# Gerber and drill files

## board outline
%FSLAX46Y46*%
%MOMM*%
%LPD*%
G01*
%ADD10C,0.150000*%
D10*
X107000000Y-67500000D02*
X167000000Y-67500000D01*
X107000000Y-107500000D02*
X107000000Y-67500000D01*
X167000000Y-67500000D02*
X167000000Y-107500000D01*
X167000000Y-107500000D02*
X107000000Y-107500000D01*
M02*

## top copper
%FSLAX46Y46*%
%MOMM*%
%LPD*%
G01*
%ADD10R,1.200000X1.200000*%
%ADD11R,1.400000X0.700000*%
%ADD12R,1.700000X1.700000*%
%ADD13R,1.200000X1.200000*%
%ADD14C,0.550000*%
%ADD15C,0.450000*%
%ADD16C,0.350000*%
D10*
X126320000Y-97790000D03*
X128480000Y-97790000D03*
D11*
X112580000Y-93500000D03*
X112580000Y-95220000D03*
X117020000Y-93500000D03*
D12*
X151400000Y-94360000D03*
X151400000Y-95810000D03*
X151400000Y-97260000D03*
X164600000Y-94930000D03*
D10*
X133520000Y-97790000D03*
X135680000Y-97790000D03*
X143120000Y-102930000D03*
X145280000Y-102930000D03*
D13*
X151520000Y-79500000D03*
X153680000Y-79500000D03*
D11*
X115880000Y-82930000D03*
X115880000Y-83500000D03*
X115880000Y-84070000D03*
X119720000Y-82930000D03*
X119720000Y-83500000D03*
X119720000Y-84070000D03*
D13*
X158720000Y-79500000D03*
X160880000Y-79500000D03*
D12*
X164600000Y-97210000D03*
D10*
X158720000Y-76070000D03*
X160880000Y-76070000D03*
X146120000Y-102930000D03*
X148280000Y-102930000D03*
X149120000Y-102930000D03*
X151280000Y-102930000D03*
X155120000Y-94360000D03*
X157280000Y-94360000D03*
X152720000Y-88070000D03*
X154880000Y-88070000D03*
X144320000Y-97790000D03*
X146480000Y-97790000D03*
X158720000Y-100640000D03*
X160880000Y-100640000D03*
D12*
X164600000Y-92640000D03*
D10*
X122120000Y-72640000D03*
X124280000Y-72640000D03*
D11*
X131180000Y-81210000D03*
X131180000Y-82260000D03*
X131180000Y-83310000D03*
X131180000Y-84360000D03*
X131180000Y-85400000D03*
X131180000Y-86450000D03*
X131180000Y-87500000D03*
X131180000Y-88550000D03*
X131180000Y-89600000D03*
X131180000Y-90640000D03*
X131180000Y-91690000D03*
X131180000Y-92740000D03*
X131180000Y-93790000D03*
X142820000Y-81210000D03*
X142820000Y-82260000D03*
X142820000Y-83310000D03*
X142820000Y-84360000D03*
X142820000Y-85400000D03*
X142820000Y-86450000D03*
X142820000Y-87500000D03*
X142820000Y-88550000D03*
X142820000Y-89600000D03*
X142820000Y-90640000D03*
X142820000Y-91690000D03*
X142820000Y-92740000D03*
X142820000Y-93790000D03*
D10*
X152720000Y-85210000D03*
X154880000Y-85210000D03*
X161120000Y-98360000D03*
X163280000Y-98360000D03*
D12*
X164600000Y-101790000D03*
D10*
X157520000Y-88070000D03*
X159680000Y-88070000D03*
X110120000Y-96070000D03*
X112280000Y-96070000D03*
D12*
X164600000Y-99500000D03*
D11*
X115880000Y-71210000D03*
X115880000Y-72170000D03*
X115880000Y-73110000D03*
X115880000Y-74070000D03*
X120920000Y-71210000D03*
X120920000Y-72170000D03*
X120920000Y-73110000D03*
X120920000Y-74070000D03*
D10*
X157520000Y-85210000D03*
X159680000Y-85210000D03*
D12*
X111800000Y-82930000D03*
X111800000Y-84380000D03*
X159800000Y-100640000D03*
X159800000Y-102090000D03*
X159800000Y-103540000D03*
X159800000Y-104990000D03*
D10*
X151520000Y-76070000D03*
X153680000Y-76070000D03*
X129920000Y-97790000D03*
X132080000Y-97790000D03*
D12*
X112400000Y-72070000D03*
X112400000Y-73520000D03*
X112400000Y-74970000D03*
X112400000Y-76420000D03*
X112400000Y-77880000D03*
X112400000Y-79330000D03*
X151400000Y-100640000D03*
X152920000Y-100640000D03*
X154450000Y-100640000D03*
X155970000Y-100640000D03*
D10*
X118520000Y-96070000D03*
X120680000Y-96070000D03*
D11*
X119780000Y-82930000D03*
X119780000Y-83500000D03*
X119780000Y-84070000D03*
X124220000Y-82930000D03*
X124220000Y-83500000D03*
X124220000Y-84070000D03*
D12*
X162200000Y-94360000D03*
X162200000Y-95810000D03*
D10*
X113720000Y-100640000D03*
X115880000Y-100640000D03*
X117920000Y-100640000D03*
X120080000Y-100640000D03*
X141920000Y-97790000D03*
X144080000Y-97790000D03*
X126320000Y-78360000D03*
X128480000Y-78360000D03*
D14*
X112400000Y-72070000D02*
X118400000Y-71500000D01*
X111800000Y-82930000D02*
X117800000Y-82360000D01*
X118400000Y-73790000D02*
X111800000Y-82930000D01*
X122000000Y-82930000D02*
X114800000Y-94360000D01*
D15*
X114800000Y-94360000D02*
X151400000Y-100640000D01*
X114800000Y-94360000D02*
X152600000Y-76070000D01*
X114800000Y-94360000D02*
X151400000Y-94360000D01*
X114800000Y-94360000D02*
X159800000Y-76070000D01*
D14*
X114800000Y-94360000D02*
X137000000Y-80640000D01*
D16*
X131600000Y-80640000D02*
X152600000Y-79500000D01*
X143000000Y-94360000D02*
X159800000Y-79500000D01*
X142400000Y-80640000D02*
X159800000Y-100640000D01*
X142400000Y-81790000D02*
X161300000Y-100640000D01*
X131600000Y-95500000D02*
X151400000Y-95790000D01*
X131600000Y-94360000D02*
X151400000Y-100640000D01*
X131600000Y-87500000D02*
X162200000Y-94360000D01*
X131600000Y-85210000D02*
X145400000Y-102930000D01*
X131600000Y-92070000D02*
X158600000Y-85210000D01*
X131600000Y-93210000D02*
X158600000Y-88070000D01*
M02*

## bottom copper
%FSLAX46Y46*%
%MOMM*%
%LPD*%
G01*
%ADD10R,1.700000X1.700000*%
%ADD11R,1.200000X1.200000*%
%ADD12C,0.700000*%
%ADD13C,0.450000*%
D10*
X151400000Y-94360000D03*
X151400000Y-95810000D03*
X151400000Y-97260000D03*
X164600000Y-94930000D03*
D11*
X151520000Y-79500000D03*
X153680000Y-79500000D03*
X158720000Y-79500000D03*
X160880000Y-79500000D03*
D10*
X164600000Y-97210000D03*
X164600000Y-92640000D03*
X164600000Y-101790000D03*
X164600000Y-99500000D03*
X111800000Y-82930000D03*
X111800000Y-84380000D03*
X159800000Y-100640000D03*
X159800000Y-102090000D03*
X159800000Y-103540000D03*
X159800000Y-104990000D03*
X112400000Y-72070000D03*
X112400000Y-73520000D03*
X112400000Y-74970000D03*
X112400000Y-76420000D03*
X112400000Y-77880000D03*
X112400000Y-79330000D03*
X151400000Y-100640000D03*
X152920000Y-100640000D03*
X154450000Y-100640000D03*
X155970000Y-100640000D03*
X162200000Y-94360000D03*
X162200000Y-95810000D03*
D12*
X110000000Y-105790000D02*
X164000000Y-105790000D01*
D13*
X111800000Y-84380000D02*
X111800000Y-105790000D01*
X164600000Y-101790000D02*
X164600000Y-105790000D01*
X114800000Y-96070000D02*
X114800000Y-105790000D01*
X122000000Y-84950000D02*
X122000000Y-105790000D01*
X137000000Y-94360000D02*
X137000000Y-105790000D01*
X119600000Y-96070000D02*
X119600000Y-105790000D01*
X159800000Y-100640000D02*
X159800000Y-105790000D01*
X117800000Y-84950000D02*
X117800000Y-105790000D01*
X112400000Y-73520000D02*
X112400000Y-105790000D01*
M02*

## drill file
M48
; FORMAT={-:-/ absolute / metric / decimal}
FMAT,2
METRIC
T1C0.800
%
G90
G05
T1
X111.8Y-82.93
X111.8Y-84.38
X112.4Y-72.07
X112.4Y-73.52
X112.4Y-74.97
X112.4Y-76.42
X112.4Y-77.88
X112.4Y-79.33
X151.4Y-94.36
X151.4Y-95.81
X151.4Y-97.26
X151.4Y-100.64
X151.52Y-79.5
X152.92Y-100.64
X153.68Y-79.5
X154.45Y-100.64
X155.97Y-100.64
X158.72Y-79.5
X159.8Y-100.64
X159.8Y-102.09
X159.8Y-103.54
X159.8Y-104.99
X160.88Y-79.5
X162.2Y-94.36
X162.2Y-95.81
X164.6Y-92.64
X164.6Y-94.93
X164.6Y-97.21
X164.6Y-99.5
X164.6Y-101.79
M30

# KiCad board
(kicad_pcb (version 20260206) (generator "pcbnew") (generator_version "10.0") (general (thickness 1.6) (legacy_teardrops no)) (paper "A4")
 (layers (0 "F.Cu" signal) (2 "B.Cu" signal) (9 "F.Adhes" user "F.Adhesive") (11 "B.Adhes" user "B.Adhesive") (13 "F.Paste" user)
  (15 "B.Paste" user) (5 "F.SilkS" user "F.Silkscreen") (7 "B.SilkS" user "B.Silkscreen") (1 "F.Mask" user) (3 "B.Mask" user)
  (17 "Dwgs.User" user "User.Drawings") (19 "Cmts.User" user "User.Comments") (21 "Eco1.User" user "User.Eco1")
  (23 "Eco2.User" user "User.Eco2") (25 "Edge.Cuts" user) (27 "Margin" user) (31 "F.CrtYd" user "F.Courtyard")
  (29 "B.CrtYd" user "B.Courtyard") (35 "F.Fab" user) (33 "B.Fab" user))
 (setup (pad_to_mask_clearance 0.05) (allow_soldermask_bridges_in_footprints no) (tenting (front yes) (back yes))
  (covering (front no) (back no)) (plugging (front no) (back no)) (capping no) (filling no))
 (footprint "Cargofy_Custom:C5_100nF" (layer "F.Cu") (at 127.4 97.79)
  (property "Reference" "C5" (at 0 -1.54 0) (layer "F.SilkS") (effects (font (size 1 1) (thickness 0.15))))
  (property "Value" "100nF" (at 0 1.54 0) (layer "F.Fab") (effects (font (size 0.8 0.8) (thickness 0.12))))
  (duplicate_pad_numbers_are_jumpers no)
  (pad "1" smd rect (at -1.08 0) (size 1.2 1.2) (layers "F.Cu" "F.Mask" "F.Paste") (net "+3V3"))
  (pad "2" smd rect (at 1.08 0) (size 1.2 1.2) (layers "F.Cu" "F.Mask" "F.Paste") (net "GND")))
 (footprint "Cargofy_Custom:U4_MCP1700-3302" (layer "F.Cu") (at 114.8 94.36)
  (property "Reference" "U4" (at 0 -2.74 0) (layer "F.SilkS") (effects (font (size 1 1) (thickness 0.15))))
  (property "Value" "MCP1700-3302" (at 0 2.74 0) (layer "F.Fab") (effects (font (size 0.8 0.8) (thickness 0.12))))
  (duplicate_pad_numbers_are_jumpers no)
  (pad "1" smd rect (at -2.22 -0.86) (size 1.4 0.7) (layers "F.Cu" "F.Mask" "F.Paste") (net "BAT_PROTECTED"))
  (pad "2" smd rect (at -2.22 0.86) (size 1.4 0.7) (layers "F.Cu" "F.Mask" "F.Paste") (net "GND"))
  (pad "3" smd rect (at 2.22 -0.86) (size 1.4 0.7) (layers "F.Cu" "F.Mask" "F.Paste") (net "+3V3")))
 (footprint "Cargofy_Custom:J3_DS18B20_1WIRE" (layer "F.Cu") (at 151.4 94.36)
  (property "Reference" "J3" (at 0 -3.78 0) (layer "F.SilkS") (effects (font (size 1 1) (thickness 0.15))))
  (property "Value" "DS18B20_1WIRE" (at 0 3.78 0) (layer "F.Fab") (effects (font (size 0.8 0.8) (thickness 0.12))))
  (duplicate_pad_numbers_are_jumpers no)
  (pad "1" thru_hole rect (at 0 0) (size 1.7 1.7) (drill 0.8) (layers "*.Cu" "*.Mask") (remove_unused_layers no) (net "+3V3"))
  (pad "2" thru_hole rect (at 0 1.45) (size 1.7 1.7) (drill 0.8) (layers "*.Cu" "*.Mask") (remove_unused_layers no) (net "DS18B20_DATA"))
  (pad "3" thru_hole rect (at 0 2.9) (size 1.7 1.7) (drill 0.8) (layers "*.Cu" "*.Mask") (remove_unused_layers no) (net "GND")))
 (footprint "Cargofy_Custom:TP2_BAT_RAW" (layer "F.Cu") (at 164.6 94.93)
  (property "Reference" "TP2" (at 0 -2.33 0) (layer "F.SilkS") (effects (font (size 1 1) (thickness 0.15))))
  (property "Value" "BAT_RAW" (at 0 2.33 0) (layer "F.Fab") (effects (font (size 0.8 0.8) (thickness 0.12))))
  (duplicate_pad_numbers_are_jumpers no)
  (pad "1" thru_hole rect (at 0 0) (size 1.7 1.7) (drill 0.8) (layers "*.Cu" "*.Mask") (remove_unused_layers no) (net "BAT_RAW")))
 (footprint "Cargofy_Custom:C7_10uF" (layer "F.Cu") (at 134.6 97.79)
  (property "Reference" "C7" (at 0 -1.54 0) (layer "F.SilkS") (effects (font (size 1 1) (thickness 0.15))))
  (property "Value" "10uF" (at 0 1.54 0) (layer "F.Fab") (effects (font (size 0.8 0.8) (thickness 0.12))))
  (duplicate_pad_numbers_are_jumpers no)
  (pad "1" smd rect (at -1.08 0) (size 1.2 1.2) (layers "F.Cu" "F.Mask" "F.Paste") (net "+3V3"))
  (pad "2" smd rect (at 1.08 0) (size 1.2 1.2) (layers "F.Cu" "F.Mask" "F.Paste") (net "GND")))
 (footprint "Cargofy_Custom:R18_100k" (layer "F.Cu") (at 144.2 102.93)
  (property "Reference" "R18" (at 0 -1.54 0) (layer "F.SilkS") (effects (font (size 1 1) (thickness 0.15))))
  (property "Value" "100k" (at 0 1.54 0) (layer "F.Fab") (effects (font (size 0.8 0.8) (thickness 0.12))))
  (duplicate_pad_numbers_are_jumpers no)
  (pad "1" smd rect (at -1.08 0) (size 1.2 1.2) (layers "F.Cu" "F.Mask" "F.Paste") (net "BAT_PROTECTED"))
  (pad "2" smd rect (at 1.08 0) (size 1.2 1.2) (layers "F.Cu" "F.Mask" "F.Paste") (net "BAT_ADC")))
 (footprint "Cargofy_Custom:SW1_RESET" (layer "F.Cu") (at 152.6 79.5)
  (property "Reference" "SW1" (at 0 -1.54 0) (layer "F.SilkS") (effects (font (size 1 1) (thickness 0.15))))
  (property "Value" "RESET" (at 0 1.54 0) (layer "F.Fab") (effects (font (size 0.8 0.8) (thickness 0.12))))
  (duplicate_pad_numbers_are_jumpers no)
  (pad "1" thru_hole rect (at -1.08 0) (size 1.2 1.2) (drill 0.8) (layers "*.Cu" "*.Mask") (remove_unused_layers no) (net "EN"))
  (pad "2" thru_hole rect (at 1.08 0) (size 1.2 1.2) (drill 0.8) (layers "*.Cu" "*.Mask") (remove_unused_layers no) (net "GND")))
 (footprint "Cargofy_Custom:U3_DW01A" (layer "F.Cu") (at 117.8 83.5)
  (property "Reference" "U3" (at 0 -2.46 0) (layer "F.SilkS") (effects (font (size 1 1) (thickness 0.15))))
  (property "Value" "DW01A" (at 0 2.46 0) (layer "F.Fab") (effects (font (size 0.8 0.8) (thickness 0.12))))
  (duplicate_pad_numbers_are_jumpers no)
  (pad "1" smd rect (at -1.92 -0.57) (size 1.4 0.7) (layers "F.Cu" "F.Mask" "F.Paste") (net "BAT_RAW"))
  (pad "2" smd rect (at -1.92 0) (size 1.4 0.7) (layers "F.Cu" "F.Mask" "F.Paste") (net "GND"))
  (pad "3" smd rect (at -1.92 0.57) (size 1.4 0.7) (layers "F.Cu" "F.Mask" "F.Paste") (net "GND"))
  (pad "4" smd rect (at 1.92 -0.57) (size 1.4 0.7) (layers "F.Cu" "F.Mask" "F.Paste") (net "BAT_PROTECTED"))
  (pad "5" smd rect (at 1.92 0) (size 1.4 0.7) (layers "F.Cu" "F.Mask" "F.Paste") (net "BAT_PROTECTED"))
  (pad "6" smd rect (at 1.92 0.57) (size 1.4 0.7) (layers "F.Cu" "F.Mask" "F.Paste") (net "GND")))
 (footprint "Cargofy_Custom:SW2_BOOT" (layer "F.Cu") (at 159.8 79.5)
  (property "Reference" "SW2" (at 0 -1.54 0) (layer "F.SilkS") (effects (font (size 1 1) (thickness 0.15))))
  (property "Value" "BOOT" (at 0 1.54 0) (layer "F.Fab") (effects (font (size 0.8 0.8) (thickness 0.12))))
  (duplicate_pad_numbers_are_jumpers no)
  (pad "1" thru_hole rect (at -1.08 0) (size 1.2 1.2) (drill 0.8) (layers "*.Cu" "*.Mask") (remove_unused_layers no) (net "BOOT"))
  (pad "2" thru_hole rect (at 1.08 0) (size 1.2 1.2) (drill 0.8) (layers "*.Cu" "*.Mask") (remove_unused_layers no) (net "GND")))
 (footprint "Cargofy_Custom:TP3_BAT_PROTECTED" (layer "F.Cu") (at 164.6 97.21)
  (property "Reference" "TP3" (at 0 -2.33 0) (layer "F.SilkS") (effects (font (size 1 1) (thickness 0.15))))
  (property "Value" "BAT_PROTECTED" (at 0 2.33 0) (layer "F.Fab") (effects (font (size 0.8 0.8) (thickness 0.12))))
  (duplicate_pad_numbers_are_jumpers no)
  (pad "1" thru_hole rect (at 0 0) (size 1.7 1.7) (drill 0.8) (layers "*.Cu" "*.Mask") (remove_unused_layers no) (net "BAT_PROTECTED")))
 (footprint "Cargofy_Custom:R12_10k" (layer "F.Cu") (at 159.8 76.07)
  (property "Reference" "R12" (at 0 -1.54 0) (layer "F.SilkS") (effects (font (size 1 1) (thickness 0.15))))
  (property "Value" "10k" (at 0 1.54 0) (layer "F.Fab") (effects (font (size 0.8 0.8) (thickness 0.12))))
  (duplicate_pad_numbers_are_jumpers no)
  (pad "1" smd rect (at -1.08 0) (size 1.2 1.2) (layers "F.Cu" "F.Mask" "F.Paste") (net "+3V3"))
  (pad "2" smd rect (at 1.08 0) (size 1.2 1.2) (layers "F.Cu" "F.Mask" "F.Paste") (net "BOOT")))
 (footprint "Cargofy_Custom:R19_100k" (layer "F.Cu") (at 147.2 102.93)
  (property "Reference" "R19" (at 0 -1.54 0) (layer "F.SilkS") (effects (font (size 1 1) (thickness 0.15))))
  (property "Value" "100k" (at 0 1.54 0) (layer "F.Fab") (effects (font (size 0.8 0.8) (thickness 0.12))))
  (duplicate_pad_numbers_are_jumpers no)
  (pad "1" smd rect (at -1.08 0) (size 1.2 1.2) (layers "F.Cu" "F.Mask" "F.Paste") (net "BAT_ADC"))
  (pad "2" smd rect (at 1.08 0) (size 1.2 1.2) (layers "F.Cu" "F.Mask" "F.Paste") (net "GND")))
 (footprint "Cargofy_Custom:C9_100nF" (layer "F.Cu") (at 150.2 102.93)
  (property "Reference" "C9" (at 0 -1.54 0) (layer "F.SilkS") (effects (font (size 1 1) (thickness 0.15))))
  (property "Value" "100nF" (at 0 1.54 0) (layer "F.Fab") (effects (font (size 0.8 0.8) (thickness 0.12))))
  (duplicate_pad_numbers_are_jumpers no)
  (pad "1" smd rect (at -1.08 0) (size 1.2 1.2) (layers "F.Cu" "F.Mask" "F.Paste") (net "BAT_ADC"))
  (pad "2" smd rect (at 1.08 0) (size 1.2 1.2) (layers "F.Cu" "F.Mask" "F.Paste") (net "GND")))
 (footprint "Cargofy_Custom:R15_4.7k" (layer "F.Cu") (at 156.2 94.36)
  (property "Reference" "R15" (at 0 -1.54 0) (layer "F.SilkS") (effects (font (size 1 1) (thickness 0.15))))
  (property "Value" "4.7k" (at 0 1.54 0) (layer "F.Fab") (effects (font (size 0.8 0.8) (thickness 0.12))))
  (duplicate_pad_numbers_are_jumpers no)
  (pad "1" smd rect (at -1.08 0) (size 1.2 1.2) (layers "F.Cu" "F.Mask" "F.Paste") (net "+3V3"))
  (pad "2" smd rect (at 1.08 0) (size 1.2 1.2) (layers "F.Cu" "F.Mask" "F.Paste") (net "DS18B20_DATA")))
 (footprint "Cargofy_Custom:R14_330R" (layer "F.Cu") (at 153.8 88.07)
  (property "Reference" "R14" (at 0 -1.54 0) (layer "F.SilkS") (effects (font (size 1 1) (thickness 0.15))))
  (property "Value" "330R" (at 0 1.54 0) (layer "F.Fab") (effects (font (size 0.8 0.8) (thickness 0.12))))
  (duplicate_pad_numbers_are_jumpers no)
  (pad "1" smd rect (at -1.08 0) (size 1.2 1.2) (layers "F.Cu" "F.Mask" "F.Paste") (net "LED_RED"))
  (pad "2" smd rect (at 1.08 0) (size 1.2 1.2) (layers "F.Cu" "F.Mask" "F.Paste") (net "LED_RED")))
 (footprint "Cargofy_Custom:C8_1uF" (layer "F.Cu") (at 145.4 97.79)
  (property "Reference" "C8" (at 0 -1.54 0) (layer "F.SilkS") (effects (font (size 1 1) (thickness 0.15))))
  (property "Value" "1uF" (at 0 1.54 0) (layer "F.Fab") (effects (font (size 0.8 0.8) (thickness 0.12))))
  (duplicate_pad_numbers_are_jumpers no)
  (pad "1" smd rect (at -1.08 0) (size 1.2 1.2) (layers "F.Cu" "F.Mask" "F.Paste") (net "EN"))
  (pad "2" smd rect (at 1.08 0) (size 1.2 1.2) (layers "F.Cu" "F.Mask" "F.Paste") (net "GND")))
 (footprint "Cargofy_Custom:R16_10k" (layer "F.Cu") (at 159.8 100.64)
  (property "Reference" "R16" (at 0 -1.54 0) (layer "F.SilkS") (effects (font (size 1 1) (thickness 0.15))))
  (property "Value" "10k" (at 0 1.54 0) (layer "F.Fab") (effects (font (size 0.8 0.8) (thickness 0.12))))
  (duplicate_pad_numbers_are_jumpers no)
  (pad "1" smd rect (at -1.08 0) (size 1.2 1.2) (layers "F.Cu" "F.Mask" "F.Paste") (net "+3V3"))
  (pad "2" smd rect (at 1.08 0) (size 1.2 1.2) (layers "F.Cu" "F.Mask" "F.Paste") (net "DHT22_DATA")))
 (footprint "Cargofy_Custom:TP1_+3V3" (layer "F.Cu") (at 164.6 92.64)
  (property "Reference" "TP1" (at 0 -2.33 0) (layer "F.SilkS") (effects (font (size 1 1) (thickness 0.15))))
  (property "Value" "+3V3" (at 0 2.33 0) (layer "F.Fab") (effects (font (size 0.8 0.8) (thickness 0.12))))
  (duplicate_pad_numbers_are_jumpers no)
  (pad "1" thru_hole rect (at 0 0) (size 1.7 1.7) (drill 0.8) (layers "*.Cu" "*.Mask") (remove_unused_layers no) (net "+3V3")))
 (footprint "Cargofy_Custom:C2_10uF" (layer "F.Cu") (at 123.2 72.64)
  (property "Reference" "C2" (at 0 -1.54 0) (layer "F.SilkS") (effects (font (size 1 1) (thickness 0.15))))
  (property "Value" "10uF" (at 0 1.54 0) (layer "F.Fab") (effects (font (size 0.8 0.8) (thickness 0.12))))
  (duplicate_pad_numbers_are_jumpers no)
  (pad "1" smd rect (at -1.08 0) (size 1.2 1.2) (layers "F.Cu" "F.Mask" "F.Paste") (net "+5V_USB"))
  (pad "2" smd rect (at 1.08 0) (size 1.2 1.2) (layers "F.Cu" "F.Mask" "F.Paste") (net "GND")))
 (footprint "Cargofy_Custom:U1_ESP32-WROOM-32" (layer "F.Cu") (at 137 87.5)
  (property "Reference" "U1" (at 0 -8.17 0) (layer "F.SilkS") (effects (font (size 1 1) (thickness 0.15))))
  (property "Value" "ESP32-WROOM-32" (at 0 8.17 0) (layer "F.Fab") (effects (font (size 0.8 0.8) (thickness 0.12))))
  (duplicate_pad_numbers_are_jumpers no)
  (pad "1" smd rect (at -5.82 -6.29) (size 1.4 0.7) (layers "F.Cu" "F.Mask" "F.Paste") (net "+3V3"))
  (pad "2" smd rect (at -5.82 -5.24) (size 1.4 0.7) (layers "F.Cu" "F.Mask" "F.Paste") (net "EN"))
  (pad "3" smd rect (at -5.82 -4.19) (size 1.4 0.7) (layers "F.Cu" "F.Mask" "F.Paste") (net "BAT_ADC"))
  (pad "4" smd rect (at -5.82 -3.14) (size 1.4 0.7) (layers "F.Cu" "F.Mask" "F.Paste") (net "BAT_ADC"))
  (pad "5" smd rect (at -5.82 -2.1) (size 1.4 0.7) (layers "F.Cu" "F.Mask" "F.Paste") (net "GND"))
  (pad "6" smd rect (at -5.82 -1.05) (size 1.4 0.7) (layers "F.Cu" "F.Mask" "F.Paste") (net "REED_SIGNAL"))
  (pad "7" smd rect (at -5.82 0) (size 1.4 0.7) (layers "F.Cu" "F.Mask" "F.Paste") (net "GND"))
  (pad "8" smd rect (at -5.82 1.05) (size 1.4 0.7) (layers "F.Cu" "F.Mask" "F.Paste") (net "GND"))
  (pad "9" smd rect (at -5.82 2.1) (size 1.4 0.7) (layers "F.Cu" "F.Mask" "F.Paste") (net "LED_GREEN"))
  (pad "10" smd rect (at -5.82 3.14) (size 1.4 0.7) (layers "F.Cu" "F.Mask" "F.Paste") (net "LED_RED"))
  (pad "11" smd rect (at -5.82 4.19) (size 1.4 0.7) (layers "F.Cu" "F.Mask" "F.Paste") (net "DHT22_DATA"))
  (pad "12" smd rect (at -5.82 5.24) (size 1.4 0.7) (layers "F.Cu" "F.Mask" "F.Paste") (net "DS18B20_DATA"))
  (pad "13" smd rect (at -5.82 6.29) (size 1.4 0.7) (layers "F.Cu" "F.Mask" "F.Paste") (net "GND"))
  (pad "14" smd rect (at 5.82 -6.29) (size 1.4 0.7) (layers "F.Cu" "F.Mask" "F.Paste") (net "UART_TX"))
  (pad "15" smd rect (at 5.82 -5.24) (size 1.4 0.7) (layers "F.Cu" "F.Mask" "F.Paste") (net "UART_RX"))
  (pad "16" smd rect (at 5.82 -4.19) (size 1.4 0.7) (layers "F.Cu" "F.Mask" "F.Paste") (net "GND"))
  (pad "17" smd rect (at 5.82 -3.14) (size 1.4 0.7) (layers "F.Cu" "F.Mask" "F.Paste") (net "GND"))
  (pad "18" smd rect (at 5.82 -2.1) (size 1.4 0.7) (layers "F.Cu" "F.Mask" "F.Paste") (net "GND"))
  (pad "19" smd rect (at 5.82 -1.05) (size 1.4 0.7) (layers "F.Cu" "F.Mask" "F.Paste") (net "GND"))
  (pad "20" smd rect (at 5.82 0) (size 1.4 0.7) (layers "F.Cu" "F.Mask" "F.Paste") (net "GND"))
  (pad "21" smd rect (at 5.82 1.05) (size 1.4 0.7) (layers "F.Cu" "F.Mask" "F.Paste") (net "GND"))
  (pad "22" smd rect (at 5.82 2.1) (size 1.4 0.7) (layers "F.Cu" "F.Mask" "F.Paste") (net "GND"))
  (pad "23" smd rect (at 5.82 3.14) (size 1.4 0.7) (layers "F.Cu" "F.Mask" "F.Paste") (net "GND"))
  (pad "24" smd rect (at 5.82 4.19) (size 1.4 0.7) (layers "F.Cu" "F.Mask" "F.Paste") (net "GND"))
  (pad "25" smd rect (at 5.82 5.24) (size 1.4 0.7) (layers "F.Cu" "F.Mask" "F.Paste") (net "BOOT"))
  (pad "26" smd rect (at 5.82 6.29) (size 1.4 0.7) (layers "F.Cu" "F.Mask" "F.Paste") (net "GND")))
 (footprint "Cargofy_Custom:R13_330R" (layer "F.Cu") (at 153.8 85.21)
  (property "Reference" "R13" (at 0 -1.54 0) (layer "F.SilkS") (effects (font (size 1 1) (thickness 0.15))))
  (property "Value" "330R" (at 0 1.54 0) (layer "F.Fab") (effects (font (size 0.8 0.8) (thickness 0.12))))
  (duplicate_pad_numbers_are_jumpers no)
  (pad "1" smd rect (at -1.08 0) (size 1.2 1.2) (layers "F.Cu" "F.Mask" "F.Paste") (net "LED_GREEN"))
  (pad "2" smd rect (at 1.08 0) (size 1.2 1.2) (layers "F.Cu" "F.Mask" "F.Paste") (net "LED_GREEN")))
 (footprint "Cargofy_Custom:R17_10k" (layer "F.Cu") (at 162.2 98.36)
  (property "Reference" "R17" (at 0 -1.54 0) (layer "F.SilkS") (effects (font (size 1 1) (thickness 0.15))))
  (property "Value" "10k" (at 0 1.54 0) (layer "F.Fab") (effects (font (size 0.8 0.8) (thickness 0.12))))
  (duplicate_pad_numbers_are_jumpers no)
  (pad "1" smd rect (at -1.08 0) (size 1.2 1.2) (layers "F.Cu" "F.Mask" "F.Paste") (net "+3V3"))
  (pad "2" smd rect (at 1.08 0) (size 1.2 1.2) (layers "F.Cu" "F.Mask" "F.Paste") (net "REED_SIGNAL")))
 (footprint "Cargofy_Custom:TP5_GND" (layer "F.Cu") (at 164.6 101.79)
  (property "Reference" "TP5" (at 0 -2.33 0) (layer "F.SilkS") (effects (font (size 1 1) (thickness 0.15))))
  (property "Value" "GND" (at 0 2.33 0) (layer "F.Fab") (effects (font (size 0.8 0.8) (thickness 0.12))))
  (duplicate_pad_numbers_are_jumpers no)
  (pad "1" thru_hole rect (at 0 0) (size 1.7 1.7) (drill 0.8) (layers "*.Cu" "*.Mask") (remove_unused_layers no) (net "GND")))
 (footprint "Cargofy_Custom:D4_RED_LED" (layer "F.Cu") (at 158.6 88.07)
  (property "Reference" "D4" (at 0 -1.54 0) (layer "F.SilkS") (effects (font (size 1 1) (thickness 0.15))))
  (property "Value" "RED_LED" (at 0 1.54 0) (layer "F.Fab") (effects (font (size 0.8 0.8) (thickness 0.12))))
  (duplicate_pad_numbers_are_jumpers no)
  (pad "1" smd rect (at -1.08 0) (size 1.2 1.2) (layers "F.Cu" "F.Mask" "F.Paste") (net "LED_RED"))
  (pad "2" smd rect (at 1.08 0) (size 1.2 1.2) (layers "F.Cu" "F.Mask" "F.Paste") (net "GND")))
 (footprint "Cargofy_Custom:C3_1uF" (layer "F.Cu") (at 111.2 96.07)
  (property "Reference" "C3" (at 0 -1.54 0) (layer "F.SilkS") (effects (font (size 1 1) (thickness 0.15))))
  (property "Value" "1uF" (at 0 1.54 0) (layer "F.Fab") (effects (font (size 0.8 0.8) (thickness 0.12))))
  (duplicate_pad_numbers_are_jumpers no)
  (pad "1" smd rect (at -1.08 0) (size 1.2 1.2) (layers "F.Cu" "F.Mask" "F.Paste") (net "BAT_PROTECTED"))
  (pad "2" smd rect (at 1.08 0) (size 1.2 1.2) (layers "F.Cu" "F.Mask" "F.Paste") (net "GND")))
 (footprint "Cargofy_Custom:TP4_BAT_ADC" (layer "F.Cu") (at 164.6 99.5)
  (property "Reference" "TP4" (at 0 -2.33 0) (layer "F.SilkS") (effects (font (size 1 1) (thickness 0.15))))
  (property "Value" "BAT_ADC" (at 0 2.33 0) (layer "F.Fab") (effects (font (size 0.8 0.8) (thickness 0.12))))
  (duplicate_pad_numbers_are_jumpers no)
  (pad "1" thru_hole rect (at 0 0) (size 1.7 1.7) (drill 0.8) (layers "*.Cu" "*.Mask") (remove_unused_layers no) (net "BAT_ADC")))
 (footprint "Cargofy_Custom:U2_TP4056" (layer "F.Cu") (at 118.4 72.64)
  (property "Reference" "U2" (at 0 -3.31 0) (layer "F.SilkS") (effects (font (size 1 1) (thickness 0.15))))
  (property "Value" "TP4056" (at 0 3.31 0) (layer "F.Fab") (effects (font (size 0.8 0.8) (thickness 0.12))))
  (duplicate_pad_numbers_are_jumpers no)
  (pad "1" smd rect (at -2.52 -1.43) (size 1.4 0.7) (layers "F.Cu" "F.Mask" "F.Paste") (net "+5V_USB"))
  (pad "2" smd rect (at -2.52 -0.47) (size 1.4 0.7) (layers "F.Cu" "F.Mask" "F.Paste") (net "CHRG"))
  (pad "3" smd rect (at -2.52 0.47) (size 1.4 0.7) (layers "F.Cu" "F.Mask" "F.Paste") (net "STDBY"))
  (pad "4" smd rect (at -2.52 1.43) (size 1.4 0.7) (layers "F.Cu" "F.Mask" "F.Paste") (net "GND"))
  (pad "5" smd rect (at 2.52 -1.43) (size 1.4 0.7) (layers "F.Cu" "F.Mask" "F.Paste") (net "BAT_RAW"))
  (pad "6" smd rect (at 2.52 -0.47) (size 1.4 0.7) (layers "F.Cu" "F.Mask" "F.Paste") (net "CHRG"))
  (pad "7" smd rect (at 2.52 0.47) (size 1.4 0.7) (layers "F.Cu" "F.Mask" "F.Paste") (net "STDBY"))
  (pad "8" smd rect (at 2.52 1.43) (size 1.4 0.7) (layers "F.Cu" "F.Mask" "F.Paste") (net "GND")))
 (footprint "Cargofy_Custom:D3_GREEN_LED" (layer "F.Cu") (at 158.6 85.21)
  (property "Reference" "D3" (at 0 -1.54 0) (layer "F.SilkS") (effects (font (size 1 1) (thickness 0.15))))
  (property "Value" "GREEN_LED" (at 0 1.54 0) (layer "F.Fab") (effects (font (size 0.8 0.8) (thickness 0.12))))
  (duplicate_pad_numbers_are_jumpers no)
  (pad "1" smd rect (at -1.08 0) (size 1.2 1.2) (layers "F.Cu" "F.Mask" "F.Paste") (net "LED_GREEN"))
  (pad "2" smd rect (at 1.08 0) (size 1.2 1.2) (layers "F.Cu" "F.Mask" "F.Paste") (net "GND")))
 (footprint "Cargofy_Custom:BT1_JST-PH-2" (layer "F.Cu") (at 111.8 82.93)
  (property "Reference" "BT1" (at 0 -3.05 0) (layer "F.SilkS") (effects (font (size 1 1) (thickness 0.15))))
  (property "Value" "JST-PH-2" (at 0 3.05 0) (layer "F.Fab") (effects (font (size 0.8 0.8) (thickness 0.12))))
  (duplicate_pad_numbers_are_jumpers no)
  (pad "1" thru_hole rect (at 0 0) (size 1.7 1.7) (drill 0.8) (layers "*.Cu" "*.Mask") (remove_unused_layers no) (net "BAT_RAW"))
  (pad "2" thru_hole rect (at 0 1.45) (size 1.7 1.7) (drill 0.8) (layers "*.Cu" "*.Mask") (remove_unused_layers no) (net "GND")))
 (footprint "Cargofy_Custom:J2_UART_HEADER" (layer "F.Cu") (at 159.8 100.64)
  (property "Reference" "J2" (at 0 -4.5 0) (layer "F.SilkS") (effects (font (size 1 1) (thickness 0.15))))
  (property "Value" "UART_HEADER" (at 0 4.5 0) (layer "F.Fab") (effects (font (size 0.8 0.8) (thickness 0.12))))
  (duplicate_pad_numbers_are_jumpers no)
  (pad "1" thru_hole rect (at 0 0) (size 1.7 1.7) (drill 0.8) (layers "*.Cu" "*.Mask") (remove_unused_layers no) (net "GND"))
  (pad "2" thru_hole rect (at 0 1.45) (size 1.7 1.7) (drill 0.8) (layers "*.Cu" "*.Mask") (remove_unused_layers no) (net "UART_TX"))
  (pad "3" thru_hole rect (at 0 2.9) (size 1.7 1.7) (drill 0.8) (layers "*.Cu" "*.Mask") (remove_unused_layers no) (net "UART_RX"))
  (pad "4" thru_hole rect (at 0 4.35) (size 1.7 1.7) (drill 0.8) (layers "*.Cu" "*.Mask") (remove_unused_layers no) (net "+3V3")))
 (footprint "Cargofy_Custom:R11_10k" (layer "F.Cu") (at 152.6 76.07)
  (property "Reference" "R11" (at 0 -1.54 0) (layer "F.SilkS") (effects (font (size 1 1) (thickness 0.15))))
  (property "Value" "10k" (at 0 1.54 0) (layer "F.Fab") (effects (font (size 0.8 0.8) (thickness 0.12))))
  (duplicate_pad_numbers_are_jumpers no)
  (pad "1" smd rect (at -1.08 0) (size 1.2 1.2) (layers "F.Cu" "F.Mask" "F.Paste") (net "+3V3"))
  (pad "2" smd rect (at 1.08 0) (size 1.2 1.2) (layers "F.Cu" "F.Mask" "F.Paste") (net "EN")))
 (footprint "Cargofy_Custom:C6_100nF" (layer "F.Cu") (at 131 97.79)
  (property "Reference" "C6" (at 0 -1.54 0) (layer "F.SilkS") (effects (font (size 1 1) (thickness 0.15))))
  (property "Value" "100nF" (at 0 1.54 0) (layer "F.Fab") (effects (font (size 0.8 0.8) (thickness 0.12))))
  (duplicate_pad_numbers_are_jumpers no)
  (pad "1" smd rect (at -1.08 0) (size 1.2 1.2) (layers "F.Cu" "F.Mask" "F.Paste") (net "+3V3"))
  (pad "2" smd rect (at 1.08 0) (size 1.2 1.2) (layers "F.Cu" "F.Mask" "F.Paste") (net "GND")))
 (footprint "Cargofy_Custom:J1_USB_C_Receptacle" (layer "F.Cu") (at 112.4 72.07)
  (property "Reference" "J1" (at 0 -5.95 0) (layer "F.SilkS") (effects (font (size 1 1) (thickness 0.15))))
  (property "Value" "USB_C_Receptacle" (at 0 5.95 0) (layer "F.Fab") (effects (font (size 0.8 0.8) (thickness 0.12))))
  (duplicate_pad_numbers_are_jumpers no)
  (pad "1" thru_hole rect (at 0 0) (size 1.7 1.7) (drill 0.8) (layers "*.Cu" "*.Mask") (remove_unused_layers no) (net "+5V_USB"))
  (pad "2" thru_hole rect (at 0 1.45) (size 1.7 1.7) (drill 0.8) (layers "*.Cu" "*.Mask") (remove_unused_layers no) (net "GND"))
  (pad "3" thru_hole rect (at 0 2.9) (size 1.7 1.7) (drill 0.8) (layers "*.Cu" "*.Mask") (remove_unused_layers no) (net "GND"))
  (pad "4" thru_hole rect (at 0 4.35) (size 1.7 1.7) (drill 0.8) (layers "*.Cu" "*.Mask") (remove_unused_layers no) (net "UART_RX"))
  (pad "5" thru_hole rect (at 0 5.81) (size 1.7 1.7) (drill 0.8) (layers "*.Cu" "*.Mask") (remove_unused_layers no) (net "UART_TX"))
  (pad "6" thru_hole rect (at 0 7.26) (size 1.7 1.7) (drill 0.8) (layers "*.Cu" "*.Mask") (remove_unused_layers no) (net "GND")))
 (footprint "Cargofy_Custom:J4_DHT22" (layer "F.Cu") (at 151.4 100.64)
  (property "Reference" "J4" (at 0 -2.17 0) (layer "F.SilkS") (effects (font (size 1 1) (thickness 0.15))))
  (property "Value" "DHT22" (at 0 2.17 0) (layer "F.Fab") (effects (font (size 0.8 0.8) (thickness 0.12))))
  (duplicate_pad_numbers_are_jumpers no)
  (pad "1" thru_hole rect (at 0 0) (size 1.7 1.7) (drill 0.8) (layers "*.Cu" "*.Mask") (remove_unused_layers no) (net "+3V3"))
  (pad "2" thru_hole rect (at 1.52 0) (size 1.7 1.7) (drill 0.8) (layers "*.Cu" "*.Mask") (remove_unused_layers no) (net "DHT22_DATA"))
  (pad "3" thru_hole rect (at 3.05 0) (size 1.7 1.7) (drill 0.8) (layers "*.Cu" "*.Mask") (remove_unused_layers no) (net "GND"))
  (pad "4" thru_hole rect (at 4.57 0) (size 1.7 1.7) (drill 0.8) (layers "*.Cu" "*.Mask") (remove_unused_layers no) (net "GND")))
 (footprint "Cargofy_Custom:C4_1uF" (layer "F.Cu") (at 119.6 96.07)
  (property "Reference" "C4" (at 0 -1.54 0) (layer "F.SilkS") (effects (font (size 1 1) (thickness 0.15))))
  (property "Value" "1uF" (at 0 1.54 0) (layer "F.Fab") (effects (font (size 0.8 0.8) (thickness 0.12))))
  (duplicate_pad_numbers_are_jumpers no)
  (pad "1" smd rect (at -1.08 0) (size 1.2 1.2) (layers "F.Cu" "F.Mask" "F.Paste") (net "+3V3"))
  (pad "2" smd rect (at 1.08 0) (size 1.2 1.2) (layers "F.Cu" "F.Mask" "F.Paste") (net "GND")))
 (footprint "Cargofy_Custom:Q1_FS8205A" (layer "F.Cu") (at 122 83.5)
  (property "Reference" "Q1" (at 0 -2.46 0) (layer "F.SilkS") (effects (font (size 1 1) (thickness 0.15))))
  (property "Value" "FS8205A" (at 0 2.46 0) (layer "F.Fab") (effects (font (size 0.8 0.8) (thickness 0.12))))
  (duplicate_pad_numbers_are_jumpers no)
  (pad "1" smd rect (at -2.22 -0.57) (size 1.4 0.7) (layers "F.Cu" "F.Mask" "F.Paste") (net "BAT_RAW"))
  (pad "2" smd rect (at -2.22 0) (size 1.4 0.7) (layers "F.Cu" "F.Mask" "F.Paste") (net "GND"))
  (pad "3" smd rect (at -2.22 0.57) (size 1.4 0.7) (layers "F.Cu" "F.Mask" "F.Paste") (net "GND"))
  (pad "4" smd rect (at 2.22 -0.57) (size 1.4 0.7) (layers "F.Cu" "F.Mask" "F.Paste") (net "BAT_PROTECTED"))
  (pad "5" smd rect (at 2.22 0) (size 1.4 0.7) (layers "F.Cu" "F.Mask" "F.Paste") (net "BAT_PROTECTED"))
  (pad "6" smd rect (at 2.22 0.57) (size 1.4 0.7) (layers "F.Cu" "F.Mask" "F.Paste") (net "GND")))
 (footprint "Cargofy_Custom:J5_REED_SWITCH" (layer "F.Cu") (at 162.2 94.36)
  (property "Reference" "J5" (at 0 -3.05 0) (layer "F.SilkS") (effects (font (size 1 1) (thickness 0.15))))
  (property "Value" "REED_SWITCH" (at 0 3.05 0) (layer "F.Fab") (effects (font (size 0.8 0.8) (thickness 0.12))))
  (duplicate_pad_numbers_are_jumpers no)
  (pad "1" thru_hole rect (at 0 0) (size 1.7 1.7) (drill 0.8) (layers "*.Cu" "*.Mask") (remove_unused_layers no) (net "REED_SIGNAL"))
  (pad "2" thru_hole rect (at 0 1.45) (size 1.7 1.7) (drill 0.8) (layers "*.Cu" "*.Mask") (remove_unused_layers no) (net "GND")))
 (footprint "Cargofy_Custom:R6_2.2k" (layer "F.Cu") (at 114.8 100.64)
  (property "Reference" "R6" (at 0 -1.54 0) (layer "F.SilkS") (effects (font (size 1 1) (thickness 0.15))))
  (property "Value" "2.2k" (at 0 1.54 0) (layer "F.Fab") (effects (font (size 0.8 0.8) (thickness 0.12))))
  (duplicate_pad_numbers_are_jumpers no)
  (pad "1" smd rect (at -1.08 0) (size 1.2 1.2) (layers "F.Cu" "F.Mask" "F.Paste") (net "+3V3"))
  (pad "2" smd rect (at 1.08 0) (size 1.2 1.2) (layers "F.Cu" "F.Mask" "F.Paste") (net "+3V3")))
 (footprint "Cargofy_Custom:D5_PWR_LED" (layer "F.Cu") (at 119 100.64)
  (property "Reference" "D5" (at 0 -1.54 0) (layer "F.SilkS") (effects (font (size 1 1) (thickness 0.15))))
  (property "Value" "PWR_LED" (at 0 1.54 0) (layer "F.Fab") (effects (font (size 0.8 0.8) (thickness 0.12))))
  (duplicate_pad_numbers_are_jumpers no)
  (pad "1" smd rect (at -1.08 0) (size 1.2 1.2) (layers "F.Cu" "F.Mask" "F.Paste") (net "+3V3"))
  (pad "2" smd rect (at 1.08 0) (size 1.2 1.2) (layers "F.Cu" "F.Mask" "F.Paste") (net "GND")))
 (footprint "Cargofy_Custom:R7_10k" (layer "F.Cu") (at 143 97.79)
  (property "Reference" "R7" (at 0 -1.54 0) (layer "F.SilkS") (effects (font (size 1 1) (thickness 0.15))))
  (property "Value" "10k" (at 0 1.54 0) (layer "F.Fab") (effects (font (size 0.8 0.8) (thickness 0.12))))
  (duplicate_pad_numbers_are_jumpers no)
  (pad "1" smd rect (at -1.08 0) (size 1.2 1.2) (layers "F.Cu" "F.Mask" "F.Paste") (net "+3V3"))
  (pad "2" smd rect (at 1.08 0) (size 1.2 1.2) (layers "F.Cu" "F.Mask" "F.Paste") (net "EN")))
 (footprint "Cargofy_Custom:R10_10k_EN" (layer "F.Cu") (at 127.4 78.36)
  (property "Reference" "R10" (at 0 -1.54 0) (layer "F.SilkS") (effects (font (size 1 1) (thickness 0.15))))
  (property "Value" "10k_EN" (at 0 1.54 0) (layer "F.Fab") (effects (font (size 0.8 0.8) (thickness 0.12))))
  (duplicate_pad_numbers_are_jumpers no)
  (pad "1" smd rect (at -1.08 0) (size 1.2 1.2) (layers "F.Cu" "F.Mask" "F.Paste") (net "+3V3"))
  (pad "2" smd rect (at 1.08 0) (size 1.2 1.2) (layers "F.Cu" "F.Mask" "F.Paste") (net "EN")))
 (gr_line (start 107 67.5) (end 167 67.5) (stroke (width 0.15) (type solid)) (layer "Edge.Cuts"))
 (gr_line (start 107 107.5) (end 107 67.5) (stroke (width 0.15) (type solid)) (layer "Edge.Cuts"))
 (gr_line (start 167 67.5) (end 167 107.5) (stroke (width 0.15) (type solid)) (layer "Edge.Cuts"))
 (gr_line (start 167 107.5) (end 107 107.5) (stroke (width 0.15) (type solid)) (layer "Edge.Cuts"))
 (segment (start 112.4 72.07) (end 118.4 71.5) (width 0.55) (layer "F.Cu") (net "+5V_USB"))
 (segment (start 111.8 82.93) (end 117.8 82.36) (width 0.55) (layer "F.Cu") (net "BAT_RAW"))
 (segment (start 118.4 73.79) (end 111.8 82.93) (width 0.55) (layer "F.Cu") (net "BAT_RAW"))
 (segment (start 122 82.93) (end 114.8 94.36) (width 0.55) (layer "F.Cu") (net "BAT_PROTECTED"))
 (segment (start 114.8 94.36) (end 151.4 100.64) (width 0.45) (layer "F.Cu") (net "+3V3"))
 (segment (start 114.8 94.36) (end 152.6 76.07) (width 0.45) (layer "F.Cu") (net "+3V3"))
 (segment (start 114.8 94.36) (end 151.4 94.36) (width 0.45) (layer "F.Cu") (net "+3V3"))
 (segment (start 114.8 94.36) (end 159.8 76.07) (width 0.45) (layer "F.Cu") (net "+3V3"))
 (segment (start 114.8 94.36) (end 137 80.64) (width 0.55) (layer "F.Cu") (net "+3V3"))
 (segment (start 110 105.79) (end 164 105.79) (width 0.7) (layer "B.Cu") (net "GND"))
 (segment (start 111.8 84.38) (end 111.8 105.79) (width 0.45) (layer "B.Cu") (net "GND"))
 (segment (start 164.6 101.79) (end 164.6 105.79) (width 0.45) (layer "B.Cu") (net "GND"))
 (segment (start 114.8 96.07) (end 114.8 105.79) (width 0.45) (layer "B.Cu") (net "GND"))
 (segment (start 122 84.95) (end 122 105.79) (width 0.45) (layer "B.Cu") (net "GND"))
 (segment (start 137 94.36) (end 137 105.79) (width 0.45) (layer "B.Cu") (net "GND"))
 (segment (start 119.6 96.07) (end 119.6 105.79) (width 0.45) (layer "B.Cu") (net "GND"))
 (segment (start 159.8 100.64) (end 159.8 105.79) (width 0.45) (layer "B.Cu") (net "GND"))
 (segment (start 117.8 84.95) (end 117.8 105.79) (width 0.45) (layer "B.Cu") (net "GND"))
 (segment (start 112.4 73.52) (end 112.4 105.79) (width 0.45) (layer "B.Cu") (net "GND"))
 (segment (start 131.6 80.64) (end 152.6 79.5) (width 0.35) (layer "F.Cu") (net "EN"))
 (segment (start 143 94.36) (end 159.8 79.5) (width 0.35) (layer "F.Cu") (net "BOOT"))
 (segment (start 142.4 80.64) (end 159.8 100.64) (width 0.35) (layer "F.Cu") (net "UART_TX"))
 (segment (start 142.4 81.79) (end 161.3 100.64) (width 0.35) (layer "F.Cu") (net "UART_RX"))
 (segment (start 131.6 95.5) (end 151.4 95.79) (width 0.35) (layer "F.Cu") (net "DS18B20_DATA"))
 (segment (start 131.6 94.36) (end 151.4 100.64) (width 0.35) (layer "F.Cu") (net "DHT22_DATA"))
 (segment (start 131.6 87.5) (end 162.2 94.36) (width 0.35) (layer "F.Cu") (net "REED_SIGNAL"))
 (segment (start 131.6 85.21) (end 145.4 102.93) (width 0.35) (layer "F.Cu") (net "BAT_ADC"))
 (segment (start 131.6 92.07) (end 158.6 85.21) (width 0.35) (layer "F.Cu") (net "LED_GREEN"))
 (segment (start 131.6 93.21) (end 158.6 88.07) (width 0.35) (layer "F.Cu") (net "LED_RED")))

